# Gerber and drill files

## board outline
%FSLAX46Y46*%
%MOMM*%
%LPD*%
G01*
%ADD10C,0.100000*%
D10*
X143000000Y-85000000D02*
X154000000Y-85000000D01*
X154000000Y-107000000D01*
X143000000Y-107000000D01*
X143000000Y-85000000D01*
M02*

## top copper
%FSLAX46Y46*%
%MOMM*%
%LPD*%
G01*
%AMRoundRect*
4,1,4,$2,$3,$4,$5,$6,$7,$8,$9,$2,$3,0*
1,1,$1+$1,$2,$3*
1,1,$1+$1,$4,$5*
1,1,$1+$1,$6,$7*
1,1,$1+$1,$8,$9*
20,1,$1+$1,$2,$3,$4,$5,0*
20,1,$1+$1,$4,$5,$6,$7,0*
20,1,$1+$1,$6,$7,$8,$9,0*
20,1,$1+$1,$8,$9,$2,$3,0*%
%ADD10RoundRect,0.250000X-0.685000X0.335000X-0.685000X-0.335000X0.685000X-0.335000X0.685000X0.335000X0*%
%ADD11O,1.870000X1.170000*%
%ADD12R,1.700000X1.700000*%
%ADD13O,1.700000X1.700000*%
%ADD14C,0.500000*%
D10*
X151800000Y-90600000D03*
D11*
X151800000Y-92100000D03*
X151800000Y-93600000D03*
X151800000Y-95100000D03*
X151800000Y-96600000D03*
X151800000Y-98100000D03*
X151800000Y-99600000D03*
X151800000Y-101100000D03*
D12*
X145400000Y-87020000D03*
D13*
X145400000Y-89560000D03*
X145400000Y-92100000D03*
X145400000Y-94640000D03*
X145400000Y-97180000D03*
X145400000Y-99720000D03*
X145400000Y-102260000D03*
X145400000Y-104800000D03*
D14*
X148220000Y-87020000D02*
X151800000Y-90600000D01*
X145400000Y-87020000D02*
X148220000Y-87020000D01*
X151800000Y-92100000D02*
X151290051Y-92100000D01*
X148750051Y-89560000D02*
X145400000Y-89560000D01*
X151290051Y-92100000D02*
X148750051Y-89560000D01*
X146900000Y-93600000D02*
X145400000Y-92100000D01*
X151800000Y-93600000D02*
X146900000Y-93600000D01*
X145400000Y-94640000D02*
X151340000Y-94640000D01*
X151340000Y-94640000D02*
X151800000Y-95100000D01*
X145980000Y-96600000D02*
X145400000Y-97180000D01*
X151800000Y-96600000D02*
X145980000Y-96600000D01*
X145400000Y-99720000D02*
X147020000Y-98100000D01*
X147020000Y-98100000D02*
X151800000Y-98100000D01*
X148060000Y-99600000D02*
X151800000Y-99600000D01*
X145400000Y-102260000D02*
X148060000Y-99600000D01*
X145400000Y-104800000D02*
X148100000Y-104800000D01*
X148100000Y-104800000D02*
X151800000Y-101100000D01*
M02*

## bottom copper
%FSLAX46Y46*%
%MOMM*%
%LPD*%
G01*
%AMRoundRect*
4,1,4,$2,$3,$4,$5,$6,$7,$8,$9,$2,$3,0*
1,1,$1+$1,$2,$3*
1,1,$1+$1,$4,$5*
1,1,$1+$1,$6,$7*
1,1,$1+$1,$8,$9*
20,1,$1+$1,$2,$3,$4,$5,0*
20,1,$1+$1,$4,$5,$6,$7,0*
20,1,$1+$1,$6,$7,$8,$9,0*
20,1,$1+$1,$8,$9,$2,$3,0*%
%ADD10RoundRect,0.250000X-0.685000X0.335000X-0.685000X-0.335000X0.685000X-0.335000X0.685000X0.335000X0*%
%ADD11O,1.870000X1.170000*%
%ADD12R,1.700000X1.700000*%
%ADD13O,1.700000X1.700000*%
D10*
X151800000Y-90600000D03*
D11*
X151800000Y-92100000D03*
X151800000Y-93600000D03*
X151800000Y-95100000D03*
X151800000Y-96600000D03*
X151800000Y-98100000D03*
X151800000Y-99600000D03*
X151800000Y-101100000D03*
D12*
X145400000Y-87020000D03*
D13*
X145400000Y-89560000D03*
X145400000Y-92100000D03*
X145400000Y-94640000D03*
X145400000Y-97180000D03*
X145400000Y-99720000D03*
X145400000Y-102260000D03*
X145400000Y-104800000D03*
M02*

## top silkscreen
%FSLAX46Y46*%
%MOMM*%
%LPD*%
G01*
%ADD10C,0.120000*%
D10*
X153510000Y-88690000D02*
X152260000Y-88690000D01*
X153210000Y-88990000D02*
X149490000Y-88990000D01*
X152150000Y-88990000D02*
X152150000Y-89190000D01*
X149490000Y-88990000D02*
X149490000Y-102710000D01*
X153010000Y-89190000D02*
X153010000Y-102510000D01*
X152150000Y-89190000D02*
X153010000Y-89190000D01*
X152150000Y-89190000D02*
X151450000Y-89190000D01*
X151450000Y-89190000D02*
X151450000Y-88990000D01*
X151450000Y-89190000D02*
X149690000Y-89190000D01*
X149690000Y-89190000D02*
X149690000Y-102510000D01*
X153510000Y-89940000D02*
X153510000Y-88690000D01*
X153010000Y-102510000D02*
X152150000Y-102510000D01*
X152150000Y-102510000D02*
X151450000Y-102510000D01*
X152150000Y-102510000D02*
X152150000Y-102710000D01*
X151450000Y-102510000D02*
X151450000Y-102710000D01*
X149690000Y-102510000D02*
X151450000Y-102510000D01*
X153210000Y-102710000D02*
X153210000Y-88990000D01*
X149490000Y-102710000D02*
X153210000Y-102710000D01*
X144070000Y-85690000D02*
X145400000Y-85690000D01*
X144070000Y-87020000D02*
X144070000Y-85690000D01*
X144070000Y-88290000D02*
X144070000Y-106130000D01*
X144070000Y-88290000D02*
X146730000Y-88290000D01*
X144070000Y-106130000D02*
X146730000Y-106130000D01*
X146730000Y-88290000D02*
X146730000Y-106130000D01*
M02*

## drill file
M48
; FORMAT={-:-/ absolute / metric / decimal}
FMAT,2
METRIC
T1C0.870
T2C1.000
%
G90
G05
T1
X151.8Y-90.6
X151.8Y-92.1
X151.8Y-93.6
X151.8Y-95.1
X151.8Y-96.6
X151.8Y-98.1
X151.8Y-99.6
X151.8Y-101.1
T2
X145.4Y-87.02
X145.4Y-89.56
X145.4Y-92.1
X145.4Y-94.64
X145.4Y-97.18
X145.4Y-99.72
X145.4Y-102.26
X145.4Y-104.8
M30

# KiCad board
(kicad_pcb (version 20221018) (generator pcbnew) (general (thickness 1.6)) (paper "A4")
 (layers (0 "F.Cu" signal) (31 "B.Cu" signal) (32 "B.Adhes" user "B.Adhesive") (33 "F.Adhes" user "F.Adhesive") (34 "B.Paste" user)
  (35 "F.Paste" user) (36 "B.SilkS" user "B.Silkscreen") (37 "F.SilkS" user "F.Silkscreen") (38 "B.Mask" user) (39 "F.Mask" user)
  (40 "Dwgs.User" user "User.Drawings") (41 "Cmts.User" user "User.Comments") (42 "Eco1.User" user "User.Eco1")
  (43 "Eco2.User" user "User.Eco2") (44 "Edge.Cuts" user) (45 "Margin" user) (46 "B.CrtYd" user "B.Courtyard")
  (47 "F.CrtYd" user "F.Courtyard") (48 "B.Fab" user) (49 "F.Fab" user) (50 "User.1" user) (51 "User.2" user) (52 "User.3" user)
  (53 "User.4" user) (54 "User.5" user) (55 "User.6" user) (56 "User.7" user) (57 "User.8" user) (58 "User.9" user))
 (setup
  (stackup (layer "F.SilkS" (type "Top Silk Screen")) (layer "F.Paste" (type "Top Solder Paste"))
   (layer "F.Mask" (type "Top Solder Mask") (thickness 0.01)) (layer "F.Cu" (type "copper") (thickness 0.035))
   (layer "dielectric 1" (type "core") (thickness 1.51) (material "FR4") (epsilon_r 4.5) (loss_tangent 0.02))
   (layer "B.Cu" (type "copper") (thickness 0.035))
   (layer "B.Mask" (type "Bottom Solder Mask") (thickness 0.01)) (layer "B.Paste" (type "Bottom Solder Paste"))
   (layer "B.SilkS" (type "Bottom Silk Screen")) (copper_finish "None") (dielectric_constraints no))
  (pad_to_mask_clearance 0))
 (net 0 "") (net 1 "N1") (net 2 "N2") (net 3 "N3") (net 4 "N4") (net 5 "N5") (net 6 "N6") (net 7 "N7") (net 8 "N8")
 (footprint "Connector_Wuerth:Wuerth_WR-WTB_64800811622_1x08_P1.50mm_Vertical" (layer "F.Cu") (at 151.8 90.6 -90)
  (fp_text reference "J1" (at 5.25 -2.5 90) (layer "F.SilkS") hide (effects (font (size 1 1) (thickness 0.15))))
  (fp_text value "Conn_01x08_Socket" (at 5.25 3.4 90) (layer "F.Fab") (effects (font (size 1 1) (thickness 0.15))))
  (fp_line (start -1.91 -1.71) (end -1.91 -0.46) (stroke (width 0.12) (type solid)) (layer "F.SilkS"))
  (fp_line (start -1.61 -1.41) (end -1.61 2.31) (stroke (width 0.12) (type solid)) (layer "F.SilkS"))
  (fp_line (start -1.61 -0.35) (end -1.41 -0.35) (stroke (width 0.12) (type solid)) (layer "F.SilkS"))
  (fp_line (start -1.61 2.31) (end 12.11 2.31) (stroke (width 0.12) (type solid)) (layer "F.SilkS"))
  (fp_line (start -1.41 -1.21) (end 11.91 -1.21) (stroke (width 0.12) (type solid)) (layer "F.SilkS"))
  (fp_line (start -1.41 -0.35) (end -1.41 -1.21) (stroke (width 0.12) (type solid)) (layer "F.SilkS"))
  (fp_line (start -1.41 -0.35) (end -1.41 0.35) (stroke (width 0.12) (type solid)) (layer "F.SilkS"))
  (fp_line (start -1.41 0.35) (end -1.61 0.35) (stroke (width 0.12) (type solid)) (layer "F.SilkS"))
  (fp_line (start -1.41 0.35) (end -1.41 2.11) (stroke (width 0.12) (type solid)) (layer "F.SilkS"))
  (fp_line (start -1.41 2.11) (end 11.91 2.11) (stroke (width 0.12) (type solid)) (layer "F.SilkS"))
  (fp_line (start -0.66 -1.71) (end -1.91 -1.71) (stroke (width 0.12) (type solid)) (layer "F.SilkS"))
  (fp_line (start 11.91 -1.21) (end 11.91 -0.35) (stroke (width 0.12) (type solid)) (layer "F.SilkS"))
  (fp_line (start 11.91 -0.35) (end 11.91 0.35) (stroke (width 0.12) (type solid)) (layer "F.SilkS"))
  (fp_line (start 11.91 -0.35) (end 12.11 -0.35) (stroke (width 0.12) (type solid)) (layer "F.SilkS"))
  (fp_line (start 11.91 0.35) (end 12.11 0.35) (stroke (width 0.12) (type solid)) (layer "F.SilkS"))
  (fp_line (start 11.91 2.11) (end 11.91 0.35) (stroke (width 0.12) (type solid)) (layer "F.SilkS"))
  (fp_line (start 12.11 -1.41) (end -1.61 -1.41) (stroke (width 0.12) (type solid)) (layer "F.SilkS"))
  (fp_line (start 12.11 2.31) (end 12.11 -1.41) (stroke (width 0.12) (type solid)) (layer "F.SilkS"))
  (pad "1" thru_hole roundrect (at 0 0 270) (size 1.17 1.87) (drill 0.87) (layers "*.Cu" "*.Mask") (roundrect_rratio 0.213675) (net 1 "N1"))
  (pad "2" thru_hole oval (at 1.5 0 270) (size 1.17 1.87) (drill 0.87) (layers "*.Cu" "*.Mask") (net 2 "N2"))
  (pad "3" thru_hole oval (at 3 0 270) (size 1.17 1.87) (drill 0.87) (layers "*.Cu" "*.Mask") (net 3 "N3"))
  (pad "4" thru_hole oval (at 4.5 0 270) (size 1.17 1.87) (drill 0.87) (layers "*.Cu" "*.Mask") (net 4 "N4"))
  (pad "5" thru_hole oval (at 6 0 270) (size 1.17 1.87) (drill 0.87) (layers "*.Cu" "*.Mask") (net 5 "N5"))
  (pad "6" thru_hole oval (at 7.5 0 270) (size 1.17 1.87) (drill 0.87) (layers "*.Cu" "*.Mask") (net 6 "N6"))
  (pad "7" thru_hole oval (at 9 0 270) (size 1.17 1.87) (drill 0.87) (layers "*.Cu" "*.Mask") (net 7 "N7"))
  (pad "8" thru_hole oval (at 10.5 0 270) (size 1.17 1.87) (drill 0.87) (layers "*.Cu" "*.Mask") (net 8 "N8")))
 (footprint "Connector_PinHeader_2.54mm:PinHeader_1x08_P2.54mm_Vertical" (layer "F.Cu") (at 145.4 87.02)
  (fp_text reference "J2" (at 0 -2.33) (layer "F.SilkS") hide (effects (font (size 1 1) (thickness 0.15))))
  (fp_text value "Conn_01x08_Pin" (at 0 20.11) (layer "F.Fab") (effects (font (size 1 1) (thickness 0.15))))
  (fp_line (start -1.33 -1.33) (end 0 -1.33) (stroke (width 0.12) (type solid)) (layer "F.SilkS"))
  (fp_line (start -1.33 0) (end -1.33 -1.33) (stroke (width 0.12) (type solid)) (layer "F.SilkS"))
  (fp_line (start -1.33 1.27) (end -1.33 19.11) (stroke (width 0.12) (type solid)) (layer "F.SilkS"))
  (fp_line (start -1.33 1.27) (end 1.33 1.27) (stroke (width 0.12) (type solid)) (layer "F.SilkS"))
  (fp_line (start -1.33 19.11) (end 1.33 19.11) (stroke (width 0.12) (type solid)) (layer "F.SilkS"))
  (fp_line (start 1.33 1.27) (end 1.33 19.11) (stroke (width 0.12) (type solid)) (layer "F.SilkS"))
  (pad "1" thru_hole rect (at 0 0) (size 1.7 1.7) (drill 1) (layers "*.Cu" "*.Mask") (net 1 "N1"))
  (pad "2" thru_hole oval (at 0 2.54) (size 1.7 1.7) (drill 1) (layers "*.Cu" "*.Mask") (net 2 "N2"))
  (pad "3" thru_hole oval (at 0 5.08) (size 1.7 1.7) (drill 1) (layers "*.Cu" "*.Mask") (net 3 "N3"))
  (pad "4" thru_hole oval (at 0 7.62) (size 1.7 1.7) (drill 1) (layers "*.Cu" "*.Mask") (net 4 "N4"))
  (pad "5" thru_hole oval (at 0 10.16) (size 1.7 1.7) (drill 1) (layers "*.Cu" "*.Mask") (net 5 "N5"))
  (pad "6" thru_hole oval (at 0 12.7) (size 1.7 1.7) (drill 1) (layers "*.Cu" "*.Mask") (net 6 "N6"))
  (pad "7" thru_hole oval (at 0 15.24) (size 1.7 1.7) (drill 1) (layers "*.Cu" "*.Mask") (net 7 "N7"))
  (pad "8" thru_hole oval (at 0 17.78) (size 1.7 1.7) (drill 1) (layers "*.Cu" "*.Mask") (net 8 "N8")))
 (gr_rect (start 143 85) (end 154 107) (stroke (width 0.1) (type default)) (fill none) (layer "Edge.Cuts"))
 (segment (start 148.22 87.02) (end 151.8 90.6) (width 0.5) (layer "F.Cu") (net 1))
 (segment (start 145.4 87.02) (end 148.22 87.02) (width 0.5) (layer "F.Cu") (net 1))
 (segment (start 151.8 92.1) (end 151.290051 92.1) (width 0.5) (layer "F.Cu") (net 2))
 (segment (start 148.750051 89.56) (end 145.4 89.56) (width 0.5) (layer "F.Cu") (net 2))
 (segment (start 151.290051 92.1) (end 148.750051 89.56) (width 0.5) (layer "F.Cu") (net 2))
 (segment (start 146.9 93.6) (end 145.4 92.1) (width 0.5) (layer "F.Cu") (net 3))
 (segment (start 151.8 93.6) (end 146.9 93.6) (width 0.5) (layer "F.Cu") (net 3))
 (segment (start 145.4 94.64) (end 151.34 94.64) (width 0.5) (layer "F.Cu") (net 4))
 (segment (start 151.34 94.64) (end 151.8 95.1) (width 0.5) (layer "F.Cu") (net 4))
 (segment (start 145.98 96.6) (end 145.4 97.18) (width 0.5) (layer "F.Cu") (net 5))
 (segment (start 151.8 96.6) (end 145.98 96.6) (width 0.5) (layer "F.Cu") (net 5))
 (segment (start 145.4 99.72) (end 147.02 98.1) (width 0.5) (layer "F.Cu") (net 6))
 (segment (start 147.02 98.1) (end 151.8 98.1) (width 0.5) (layer "F.Cu") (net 6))
 (segment (start 148.06 99.6) (end 151.8 99.6) (width 0.5) (layer "F.Cu") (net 7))
 (segment (start 145.4 102.26) (end 148.06 99.6) (width 0.5) (layer "F.Cu") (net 7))
 (segment (start 145.4 104.8) (end 148.1 104.8) (width 0.5) (layer "F.Cu") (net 8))
 (segment (start 148.1 104.8) (end 151.8 101.1) (width 0.5) (layer "F.Cu") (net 8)))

